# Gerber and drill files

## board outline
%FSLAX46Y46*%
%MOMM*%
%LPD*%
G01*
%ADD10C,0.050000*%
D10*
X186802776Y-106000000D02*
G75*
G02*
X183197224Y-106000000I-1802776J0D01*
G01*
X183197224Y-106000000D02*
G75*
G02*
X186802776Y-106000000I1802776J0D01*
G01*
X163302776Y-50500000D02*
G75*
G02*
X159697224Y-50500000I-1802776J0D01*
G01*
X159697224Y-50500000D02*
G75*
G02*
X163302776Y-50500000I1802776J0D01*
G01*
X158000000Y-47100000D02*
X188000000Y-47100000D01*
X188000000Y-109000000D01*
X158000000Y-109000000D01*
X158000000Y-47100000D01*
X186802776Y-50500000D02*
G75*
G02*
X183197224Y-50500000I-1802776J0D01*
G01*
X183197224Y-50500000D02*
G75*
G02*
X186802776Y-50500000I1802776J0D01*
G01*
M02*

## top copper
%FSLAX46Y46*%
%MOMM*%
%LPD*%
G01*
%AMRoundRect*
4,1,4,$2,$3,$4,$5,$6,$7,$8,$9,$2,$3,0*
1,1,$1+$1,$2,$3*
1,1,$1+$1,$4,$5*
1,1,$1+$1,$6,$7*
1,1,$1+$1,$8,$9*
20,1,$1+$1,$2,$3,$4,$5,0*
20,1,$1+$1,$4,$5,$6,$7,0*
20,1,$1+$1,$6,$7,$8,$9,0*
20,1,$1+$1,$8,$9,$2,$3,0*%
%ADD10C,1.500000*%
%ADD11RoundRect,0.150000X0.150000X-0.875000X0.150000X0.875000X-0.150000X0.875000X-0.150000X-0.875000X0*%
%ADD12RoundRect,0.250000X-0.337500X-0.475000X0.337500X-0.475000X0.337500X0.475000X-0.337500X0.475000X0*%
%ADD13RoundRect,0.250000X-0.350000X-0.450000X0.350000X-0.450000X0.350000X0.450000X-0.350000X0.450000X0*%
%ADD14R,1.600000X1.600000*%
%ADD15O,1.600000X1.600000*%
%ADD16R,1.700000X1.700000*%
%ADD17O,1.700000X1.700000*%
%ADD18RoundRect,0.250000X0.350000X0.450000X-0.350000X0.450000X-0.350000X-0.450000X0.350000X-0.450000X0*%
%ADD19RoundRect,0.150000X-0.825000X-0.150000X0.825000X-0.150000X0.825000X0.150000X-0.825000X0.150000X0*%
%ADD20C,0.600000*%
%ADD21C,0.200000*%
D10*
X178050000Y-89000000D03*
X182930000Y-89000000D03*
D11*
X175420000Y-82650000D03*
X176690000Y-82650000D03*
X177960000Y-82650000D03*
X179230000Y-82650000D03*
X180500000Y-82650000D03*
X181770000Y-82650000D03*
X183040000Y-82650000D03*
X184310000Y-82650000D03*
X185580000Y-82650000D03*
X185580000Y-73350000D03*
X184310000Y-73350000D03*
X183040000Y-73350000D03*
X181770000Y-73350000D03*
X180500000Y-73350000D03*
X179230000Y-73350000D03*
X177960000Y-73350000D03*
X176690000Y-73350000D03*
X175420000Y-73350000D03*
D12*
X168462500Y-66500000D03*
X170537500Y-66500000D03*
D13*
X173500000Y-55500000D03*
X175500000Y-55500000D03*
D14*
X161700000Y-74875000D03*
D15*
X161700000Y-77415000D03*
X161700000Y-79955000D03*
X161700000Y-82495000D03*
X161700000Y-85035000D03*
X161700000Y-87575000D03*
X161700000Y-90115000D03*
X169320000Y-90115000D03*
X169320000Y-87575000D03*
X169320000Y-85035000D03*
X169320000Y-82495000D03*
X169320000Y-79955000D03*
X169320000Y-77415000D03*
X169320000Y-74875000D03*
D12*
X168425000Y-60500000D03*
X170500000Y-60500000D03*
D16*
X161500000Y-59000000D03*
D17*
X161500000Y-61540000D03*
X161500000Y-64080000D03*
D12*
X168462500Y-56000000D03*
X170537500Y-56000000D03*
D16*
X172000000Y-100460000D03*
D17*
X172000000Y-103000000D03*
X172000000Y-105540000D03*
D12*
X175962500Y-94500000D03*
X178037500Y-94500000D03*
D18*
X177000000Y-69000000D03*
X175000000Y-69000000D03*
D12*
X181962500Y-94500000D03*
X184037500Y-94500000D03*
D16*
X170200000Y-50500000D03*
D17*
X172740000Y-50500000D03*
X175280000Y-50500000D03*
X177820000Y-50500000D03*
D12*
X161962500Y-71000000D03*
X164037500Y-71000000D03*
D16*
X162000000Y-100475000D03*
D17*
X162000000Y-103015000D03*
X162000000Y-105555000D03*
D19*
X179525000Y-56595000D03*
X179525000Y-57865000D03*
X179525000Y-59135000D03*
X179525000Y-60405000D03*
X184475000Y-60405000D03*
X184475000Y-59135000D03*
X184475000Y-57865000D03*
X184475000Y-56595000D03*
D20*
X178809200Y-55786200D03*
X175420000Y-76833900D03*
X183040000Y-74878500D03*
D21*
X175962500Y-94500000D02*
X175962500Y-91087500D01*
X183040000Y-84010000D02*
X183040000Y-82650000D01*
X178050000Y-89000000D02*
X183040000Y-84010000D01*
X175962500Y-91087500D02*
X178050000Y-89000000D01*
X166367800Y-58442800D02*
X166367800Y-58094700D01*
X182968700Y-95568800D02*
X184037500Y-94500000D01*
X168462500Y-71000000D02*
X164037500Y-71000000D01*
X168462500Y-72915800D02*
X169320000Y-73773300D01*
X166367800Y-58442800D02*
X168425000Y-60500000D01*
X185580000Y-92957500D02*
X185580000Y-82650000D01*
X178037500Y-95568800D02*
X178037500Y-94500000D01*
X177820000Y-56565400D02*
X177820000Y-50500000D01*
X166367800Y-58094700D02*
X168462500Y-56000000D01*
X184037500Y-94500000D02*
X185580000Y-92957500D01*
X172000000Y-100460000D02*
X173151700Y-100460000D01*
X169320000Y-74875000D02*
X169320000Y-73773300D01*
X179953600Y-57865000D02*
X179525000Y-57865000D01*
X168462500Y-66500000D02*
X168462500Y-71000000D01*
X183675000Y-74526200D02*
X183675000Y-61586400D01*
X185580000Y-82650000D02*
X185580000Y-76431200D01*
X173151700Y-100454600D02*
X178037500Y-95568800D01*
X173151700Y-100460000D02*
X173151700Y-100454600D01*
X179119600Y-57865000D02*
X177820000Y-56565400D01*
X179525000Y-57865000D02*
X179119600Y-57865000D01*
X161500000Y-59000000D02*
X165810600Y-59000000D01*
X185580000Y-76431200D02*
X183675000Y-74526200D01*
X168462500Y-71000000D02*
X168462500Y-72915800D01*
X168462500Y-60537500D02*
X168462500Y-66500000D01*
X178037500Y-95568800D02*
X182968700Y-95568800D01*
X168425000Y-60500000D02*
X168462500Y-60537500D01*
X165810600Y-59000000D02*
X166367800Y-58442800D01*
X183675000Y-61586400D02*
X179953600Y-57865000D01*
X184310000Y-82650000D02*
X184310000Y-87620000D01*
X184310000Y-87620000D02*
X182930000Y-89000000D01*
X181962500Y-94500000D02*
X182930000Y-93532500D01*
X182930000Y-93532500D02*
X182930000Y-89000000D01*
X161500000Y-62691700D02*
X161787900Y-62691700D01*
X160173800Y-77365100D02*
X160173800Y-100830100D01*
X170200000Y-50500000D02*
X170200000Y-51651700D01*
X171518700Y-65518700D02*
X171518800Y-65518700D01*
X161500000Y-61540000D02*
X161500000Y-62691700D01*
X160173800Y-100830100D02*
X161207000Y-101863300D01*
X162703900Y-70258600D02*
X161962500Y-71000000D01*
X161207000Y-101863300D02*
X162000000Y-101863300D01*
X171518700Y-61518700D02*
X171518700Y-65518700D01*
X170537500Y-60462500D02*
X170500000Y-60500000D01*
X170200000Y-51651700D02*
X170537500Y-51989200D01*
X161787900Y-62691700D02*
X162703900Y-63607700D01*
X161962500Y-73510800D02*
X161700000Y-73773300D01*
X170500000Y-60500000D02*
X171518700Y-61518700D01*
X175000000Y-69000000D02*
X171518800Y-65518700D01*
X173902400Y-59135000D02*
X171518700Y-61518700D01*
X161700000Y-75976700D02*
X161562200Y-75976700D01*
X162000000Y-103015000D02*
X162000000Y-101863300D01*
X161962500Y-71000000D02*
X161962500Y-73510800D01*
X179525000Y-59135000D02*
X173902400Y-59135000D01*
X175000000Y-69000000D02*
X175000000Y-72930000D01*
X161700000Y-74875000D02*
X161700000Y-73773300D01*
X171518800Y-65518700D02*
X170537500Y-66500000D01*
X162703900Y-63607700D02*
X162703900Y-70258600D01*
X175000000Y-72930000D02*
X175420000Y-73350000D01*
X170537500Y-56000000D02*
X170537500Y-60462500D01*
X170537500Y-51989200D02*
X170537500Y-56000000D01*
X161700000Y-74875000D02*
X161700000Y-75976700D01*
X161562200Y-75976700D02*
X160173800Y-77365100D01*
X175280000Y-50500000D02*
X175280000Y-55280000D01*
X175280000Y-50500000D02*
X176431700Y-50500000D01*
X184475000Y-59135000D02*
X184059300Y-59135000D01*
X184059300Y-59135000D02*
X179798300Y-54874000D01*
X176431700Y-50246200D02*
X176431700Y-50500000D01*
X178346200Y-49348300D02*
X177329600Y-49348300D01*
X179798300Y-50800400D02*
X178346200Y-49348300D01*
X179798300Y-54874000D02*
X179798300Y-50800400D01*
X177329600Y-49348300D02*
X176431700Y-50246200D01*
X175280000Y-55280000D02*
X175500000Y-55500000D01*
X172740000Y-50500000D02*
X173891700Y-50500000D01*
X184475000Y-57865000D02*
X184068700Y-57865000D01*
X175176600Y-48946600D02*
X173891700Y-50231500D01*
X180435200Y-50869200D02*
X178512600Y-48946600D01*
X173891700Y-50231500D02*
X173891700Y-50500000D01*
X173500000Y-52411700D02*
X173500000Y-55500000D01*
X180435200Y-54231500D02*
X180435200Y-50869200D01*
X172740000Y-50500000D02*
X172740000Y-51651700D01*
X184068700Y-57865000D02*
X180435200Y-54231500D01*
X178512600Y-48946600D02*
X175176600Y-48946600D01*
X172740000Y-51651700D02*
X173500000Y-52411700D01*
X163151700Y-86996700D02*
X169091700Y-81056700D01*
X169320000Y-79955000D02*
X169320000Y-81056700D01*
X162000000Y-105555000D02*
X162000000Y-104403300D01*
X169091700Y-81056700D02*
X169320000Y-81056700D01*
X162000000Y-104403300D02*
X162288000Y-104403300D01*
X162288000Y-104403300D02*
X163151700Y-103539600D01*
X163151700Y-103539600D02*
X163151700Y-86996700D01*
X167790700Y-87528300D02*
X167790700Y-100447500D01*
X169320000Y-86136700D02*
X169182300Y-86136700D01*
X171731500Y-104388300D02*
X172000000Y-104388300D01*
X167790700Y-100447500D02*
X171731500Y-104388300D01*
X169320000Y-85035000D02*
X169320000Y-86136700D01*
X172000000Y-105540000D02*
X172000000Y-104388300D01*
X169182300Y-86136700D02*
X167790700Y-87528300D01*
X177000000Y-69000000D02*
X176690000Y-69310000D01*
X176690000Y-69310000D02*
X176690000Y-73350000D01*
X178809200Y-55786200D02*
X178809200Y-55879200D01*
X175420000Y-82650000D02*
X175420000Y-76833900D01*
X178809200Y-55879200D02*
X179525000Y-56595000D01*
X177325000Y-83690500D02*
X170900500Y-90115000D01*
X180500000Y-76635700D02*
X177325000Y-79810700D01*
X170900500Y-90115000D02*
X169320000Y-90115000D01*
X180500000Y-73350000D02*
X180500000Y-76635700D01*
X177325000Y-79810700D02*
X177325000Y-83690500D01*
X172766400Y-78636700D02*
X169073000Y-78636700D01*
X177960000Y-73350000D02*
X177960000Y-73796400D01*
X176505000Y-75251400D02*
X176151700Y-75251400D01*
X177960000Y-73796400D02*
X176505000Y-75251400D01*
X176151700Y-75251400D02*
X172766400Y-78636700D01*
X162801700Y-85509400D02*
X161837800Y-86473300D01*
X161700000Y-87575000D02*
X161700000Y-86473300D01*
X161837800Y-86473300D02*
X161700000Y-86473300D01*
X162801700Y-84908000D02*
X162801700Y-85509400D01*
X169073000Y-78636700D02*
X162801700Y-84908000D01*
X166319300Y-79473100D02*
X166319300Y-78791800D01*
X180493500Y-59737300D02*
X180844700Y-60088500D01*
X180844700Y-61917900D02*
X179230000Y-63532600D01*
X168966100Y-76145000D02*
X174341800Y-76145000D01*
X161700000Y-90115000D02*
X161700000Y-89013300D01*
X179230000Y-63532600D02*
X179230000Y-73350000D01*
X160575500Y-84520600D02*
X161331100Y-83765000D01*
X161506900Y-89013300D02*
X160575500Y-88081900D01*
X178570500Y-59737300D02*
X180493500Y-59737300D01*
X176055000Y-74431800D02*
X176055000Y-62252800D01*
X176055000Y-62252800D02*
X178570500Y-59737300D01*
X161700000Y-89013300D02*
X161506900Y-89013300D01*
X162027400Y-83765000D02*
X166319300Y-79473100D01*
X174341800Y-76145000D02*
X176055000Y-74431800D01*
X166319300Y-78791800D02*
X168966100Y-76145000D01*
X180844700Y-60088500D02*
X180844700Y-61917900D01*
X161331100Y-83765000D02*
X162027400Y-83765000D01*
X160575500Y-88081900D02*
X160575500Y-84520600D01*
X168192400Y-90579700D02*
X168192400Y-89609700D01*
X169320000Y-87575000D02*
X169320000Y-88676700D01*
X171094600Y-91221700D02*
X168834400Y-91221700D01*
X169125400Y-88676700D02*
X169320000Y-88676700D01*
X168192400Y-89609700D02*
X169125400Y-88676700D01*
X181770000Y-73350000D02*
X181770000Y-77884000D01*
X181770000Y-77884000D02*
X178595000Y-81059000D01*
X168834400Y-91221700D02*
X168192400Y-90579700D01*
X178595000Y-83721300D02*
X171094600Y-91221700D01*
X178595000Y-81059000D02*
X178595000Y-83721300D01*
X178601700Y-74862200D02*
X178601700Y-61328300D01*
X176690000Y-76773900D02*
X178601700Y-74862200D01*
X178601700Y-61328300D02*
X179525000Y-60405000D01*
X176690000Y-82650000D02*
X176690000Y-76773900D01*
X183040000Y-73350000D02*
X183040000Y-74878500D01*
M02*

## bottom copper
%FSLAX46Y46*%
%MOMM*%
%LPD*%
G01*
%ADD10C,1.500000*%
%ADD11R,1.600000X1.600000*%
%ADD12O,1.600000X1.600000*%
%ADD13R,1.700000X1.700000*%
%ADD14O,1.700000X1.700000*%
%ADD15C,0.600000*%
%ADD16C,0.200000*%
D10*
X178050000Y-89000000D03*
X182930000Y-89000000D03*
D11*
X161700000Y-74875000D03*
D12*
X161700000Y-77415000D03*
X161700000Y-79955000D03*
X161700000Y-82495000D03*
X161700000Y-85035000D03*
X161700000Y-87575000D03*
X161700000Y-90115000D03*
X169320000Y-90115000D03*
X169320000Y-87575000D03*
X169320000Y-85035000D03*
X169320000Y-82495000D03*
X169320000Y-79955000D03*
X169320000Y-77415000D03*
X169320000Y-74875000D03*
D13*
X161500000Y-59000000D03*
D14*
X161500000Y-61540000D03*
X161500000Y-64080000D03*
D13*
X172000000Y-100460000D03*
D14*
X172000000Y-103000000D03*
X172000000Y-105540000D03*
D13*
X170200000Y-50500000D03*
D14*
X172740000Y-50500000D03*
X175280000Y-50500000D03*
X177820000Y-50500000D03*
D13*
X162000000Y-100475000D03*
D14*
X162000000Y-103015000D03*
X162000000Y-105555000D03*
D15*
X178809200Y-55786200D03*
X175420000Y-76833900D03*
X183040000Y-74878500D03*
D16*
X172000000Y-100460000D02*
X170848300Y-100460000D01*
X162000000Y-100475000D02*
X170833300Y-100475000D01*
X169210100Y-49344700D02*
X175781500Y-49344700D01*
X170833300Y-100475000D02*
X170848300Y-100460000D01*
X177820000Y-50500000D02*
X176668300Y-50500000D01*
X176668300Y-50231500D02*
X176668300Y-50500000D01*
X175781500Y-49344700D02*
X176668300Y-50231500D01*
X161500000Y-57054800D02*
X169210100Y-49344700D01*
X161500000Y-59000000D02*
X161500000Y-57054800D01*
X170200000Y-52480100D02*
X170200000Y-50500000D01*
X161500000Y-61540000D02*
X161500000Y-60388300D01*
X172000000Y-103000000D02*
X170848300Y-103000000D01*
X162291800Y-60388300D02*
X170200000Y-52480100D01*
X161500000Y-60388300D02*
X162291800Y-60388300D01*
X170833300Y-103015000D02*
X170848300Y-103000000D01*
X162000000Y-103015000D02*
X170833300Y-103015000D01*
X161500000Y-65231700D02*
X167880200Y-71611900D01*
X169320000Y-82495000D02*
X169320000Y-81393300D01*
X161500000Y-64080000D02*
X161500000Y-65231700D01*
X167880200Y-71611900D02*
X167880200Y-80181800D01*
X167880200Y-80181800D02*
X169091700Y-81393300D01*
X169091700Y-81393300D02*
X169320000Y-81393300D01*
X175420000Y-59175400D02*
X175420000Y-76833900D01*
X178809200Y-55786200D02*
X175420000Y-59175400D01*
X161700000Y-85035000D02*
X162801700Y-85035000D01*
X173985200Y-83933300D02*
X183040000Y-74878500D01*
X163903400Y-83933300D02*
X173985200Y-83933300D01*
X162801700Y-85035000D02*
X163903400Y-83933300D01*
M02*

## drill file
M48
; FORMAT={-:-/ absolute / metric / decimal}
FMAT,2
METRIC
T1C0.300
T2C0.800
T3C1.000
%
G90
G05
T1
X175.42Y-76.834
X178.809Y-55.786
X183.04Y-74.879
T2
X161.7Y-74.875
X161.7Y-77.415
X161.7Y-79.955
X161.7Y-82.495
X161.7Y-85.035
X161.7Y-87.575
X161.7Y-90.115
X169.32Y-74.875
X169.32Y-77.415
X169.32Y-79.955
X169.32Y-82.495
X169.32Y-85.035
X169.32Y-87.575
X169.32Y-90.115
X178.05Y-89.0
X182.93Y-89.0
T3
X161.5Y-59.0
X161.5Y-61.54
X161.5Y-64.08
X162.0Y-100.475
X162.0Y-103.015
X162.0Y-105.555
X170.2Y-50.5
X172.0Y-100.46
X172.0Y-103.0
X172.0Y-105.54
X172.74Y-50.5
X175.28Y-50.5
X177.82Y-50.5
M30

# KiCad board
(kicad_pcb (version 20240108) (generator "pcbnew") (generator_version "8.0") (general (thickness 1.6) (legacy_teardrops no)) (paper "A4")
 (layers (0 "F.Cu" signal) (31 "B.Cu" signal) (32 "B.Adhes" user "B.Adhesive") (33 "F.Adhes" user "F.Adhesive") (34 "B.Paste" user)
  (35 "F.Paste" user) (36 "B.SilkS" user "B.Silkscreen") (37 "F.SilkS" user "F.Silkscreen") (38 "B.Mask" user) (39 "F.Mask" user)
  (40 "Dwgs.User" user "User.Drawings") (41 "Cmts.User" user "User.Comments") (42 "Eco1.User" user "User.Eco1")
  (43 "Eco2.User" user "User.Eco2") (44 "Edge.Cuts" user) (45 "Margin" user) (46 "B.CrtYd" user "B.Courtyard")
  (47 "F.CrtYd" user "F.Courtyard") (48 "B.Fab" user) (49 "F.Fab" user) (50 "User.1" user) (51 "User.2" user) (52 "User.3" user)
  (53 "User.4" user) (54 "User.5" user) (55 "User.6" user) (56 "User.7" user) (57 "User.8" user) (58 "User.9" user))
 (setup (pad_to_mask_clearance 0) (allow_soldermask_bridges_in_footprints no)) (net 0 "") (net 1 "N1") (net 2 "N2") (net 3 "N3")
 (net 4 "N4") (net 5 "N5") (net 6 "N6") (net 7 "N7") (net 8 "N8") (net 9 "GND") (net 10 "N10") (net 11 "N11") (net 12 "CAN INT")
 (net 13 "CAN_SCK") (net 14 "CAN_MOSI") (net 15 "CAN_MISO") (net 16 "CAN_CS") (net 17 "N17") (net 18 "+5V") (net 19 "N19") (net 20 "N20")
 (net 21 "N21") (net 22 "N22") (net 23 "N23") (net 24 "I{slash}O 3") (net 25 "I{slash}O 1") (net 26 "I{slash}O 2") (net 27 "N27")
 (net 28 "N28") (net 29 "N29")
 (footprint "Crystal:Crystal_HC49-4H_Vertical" (layer "F.Cu") (at 178.05 89)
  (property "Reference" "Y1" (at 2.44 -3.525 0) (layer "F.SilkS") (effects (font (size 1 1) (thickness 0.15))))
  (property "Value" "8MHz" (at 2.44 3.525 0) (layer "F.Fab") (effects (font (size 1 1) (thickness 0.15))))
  (pad "1" thru_hole circle (at 0 0) (size 1.5 1.5) (drill 0.8) (layers "*.Cu" "*.Mask") (remove_unused_layers no) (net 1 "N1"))
  (pad "2" thru_hole circle (at 4.88 0) (size 1.5 1.5) (drill 0.8) (layers "*.Cu" "*.Mask") (remove_unused_layers no) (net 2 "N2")))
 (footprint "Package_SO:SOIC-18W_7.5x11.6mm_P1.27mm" (layer "F.Cu") (at 180.5 78 90)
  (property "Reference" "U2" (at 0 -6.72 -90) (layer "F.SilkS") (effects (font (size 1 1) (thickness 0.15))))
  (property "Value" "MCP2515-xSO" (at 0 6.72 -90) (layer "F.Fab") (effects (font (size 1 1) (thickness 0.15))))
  (pad "1" smd roundrect (at -4.65 -5.08 90) (size 2.05 0.6) (layers "F.Cu" "F.Paste" "F.Mask") (roundrect_rratio 0.25) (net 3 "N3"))
  (pad "2" smd roundrect (at -4.65 -3.81 90) (size 2.05 0.6) (layers "F.Cu" "F.Paste" "F.Mask") (roundrect_rratio 0.25) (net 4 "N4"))
  (pad "3" smd roundrect (at -4.65 -2.54 90) (size 2.05 0.6) (layers "F.Cu" "F.Paste" "F.Mask") (roundrect_rratio 0.25) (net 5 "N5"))
  (pad "4" smd roundrect (at -4.65 -1.27 90) (size 2.05 0.6) (layers "F.Cu" "F.Paste" "F.Mask") (roundrect_rratio 0.25) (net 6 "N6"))
  (pad "5" smd roundrect (at -4.65 0 90) (size 2.05 0.6) (layers "F.Cu" "F.Paste" "F.Mask") (roundrect_rratio 0.25) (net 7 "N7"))
  (pad "6" smd roundrect (at -4.65 1.27 90) (size 2.05 0.6) (layers "F.Cu" "F.Paste" "F.Mask") (roundrect_rratio 0.25) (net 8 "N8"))
  (pad "7" smd roundrect (at -4.65 2.54 90) (size 2.05 0.6) (layers "F.Cu" "F.Paste" "F.Mask") (roundrect_rratio 0.25) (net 1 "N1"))
  (pad "8" smd roundrect (at -4.65 3.81 90) (size 2.05 0.6) (layers "F.Cu" "F.Paste" "F.Mask") (roundrect_rratio 0.25) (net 2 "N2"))
  (pad "9" smd roundrect (at -4.65 5.08 90) (size 2.05 0.6) (layers "F.Cu" "F.Paste" "F.Mask") (roundrect_rratio 0.25) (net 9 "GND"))
  (pad "10" smd roundrect (at 4.65 5.08 90) (size 2.05 0.6) (layers "F.Cu" "F.Paste" "F.Mask") (roundrect_rratio 0.25) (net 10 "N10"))
  (pad "11" smd roundrect (at 4.65 3.81 90) (size 2.05 0.6) (layers "F.Cu" "F.Paste" "F.Mask") (roundrect_rratio 0.25) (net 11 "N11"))
  (pad "12" smd roundrect (at 4.65 2.54 90) (size 2.05 0.6) (layers "F.Cu" "F.Paste" "F.Mask") (roundrect_rratio 0.25) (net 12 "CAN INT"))
  (pad "13" smd roundrect (at 4.65 1.27 90) (size 2.05 0.6) (layers "F.Cu" "F.Paste" "F.Mask") (roundrect_rratio 0.25) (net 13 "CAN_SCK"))
  (pad "14" smd roundrect (at 4.65 0 90) (size 2.05 0.6) (layers "F.Cu" "F.Paste" "F.Mask") (roundrect_rratio 0.25) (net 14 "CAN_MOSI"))
  (pad "15" smd roundrect (at 4.65 -1.27 90) (size 2.05 0.6) (layers "F.Cu" "F.Paste" "F.Mask") (roundrect_rratio 0.25) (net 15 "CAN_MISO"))
  (pad "16" smd roundrect (at 4.65 -2.54 90) (size 2.05 0.6) (layers "F.Cu" "F.Paste" "F.Mask") (roundrect_rratio 0.25) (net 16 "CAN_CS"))
  (pad "17" smd roundrect (at 4.65 -3.81 90) (size 2.05 0.6) (layers "F.Cu" "F.Paste" "F.Mask") (roundrect_rratio 0.25) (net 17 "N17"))
  (pad "18" smd roundrect (at 4.65 -5.08 90) (size 2.05 0.6) (layers "F.Cu" "F.Paste" "F.Mask") (roundrect_rratio 0.25) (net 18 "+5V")))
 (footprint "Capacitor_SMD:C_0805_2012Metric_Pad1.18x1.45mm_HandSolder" (layer "F.Cu") (at 169.5 66.5)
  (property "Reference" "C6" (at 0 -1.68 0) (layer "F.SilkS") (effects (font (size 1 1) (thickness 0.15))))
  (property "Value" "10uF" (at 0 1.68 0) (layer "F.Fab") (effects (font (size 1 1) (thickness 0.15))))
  (pad "1" smd roundrect (at -1.0375 0) (size 1.175 1.45) (layers "F.Cu" "F.Paste" "F.Mask") (roundrect_rratio 0.212766) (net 9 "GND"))
  (pad "2" smd roundrect (at 1.0375 0) (size 1.175 1.45) (layers "F.Cu" "F.Paste" "F.Mask") (roundrect_rratio 0.212766) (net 18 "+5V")))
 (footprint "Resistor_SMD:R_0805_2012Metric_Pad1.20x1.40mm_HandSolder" (layer "F.Cu") (at 174.5 55.5)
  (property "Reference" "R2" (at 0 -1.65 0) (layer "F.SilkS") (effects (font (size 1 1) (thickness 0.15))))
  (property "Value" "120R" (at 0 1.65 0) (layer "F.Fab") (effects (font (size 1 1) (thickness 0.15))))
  (pad "1" smd roundrect (at -1 0) (size 1.2 1.4) (layers "F.Cu" "F.Paste" "F.Mask") (roundrect_rratio 0.208333) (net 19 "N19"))
  (pad "2" smd roundrect (at 1 0) (size 1.2 1.4) (layers "F.Cu" "F.Paste" "F.Mask") (roundrect_rratio 0.208333) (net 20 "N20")))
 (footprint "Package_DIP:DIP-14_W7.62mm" (layer "F.Cu") (at 161.7 74.875)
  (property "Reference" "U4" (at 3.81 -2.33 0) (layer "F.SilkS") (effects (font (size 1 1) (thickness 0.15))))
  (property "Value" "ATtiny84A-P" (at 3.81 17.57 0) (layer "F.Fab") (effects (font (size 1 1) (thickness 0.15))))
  (pad "1" thru_hole rect (at 0 0) (size 1.6 1.6) (drill 0.8) (layers "*.Cu" "*.Mask") (remove_unused_layers no) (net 18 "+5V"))
  (pad "2" thru_hole oval (at 0 2.54) (size 1.6 1.6) (drill 0.8) (layers "*.Cu" "*.Mask") (remove_unused_layers no) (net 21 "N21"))
  (pad "3" thru_hole oval (at 0 5.08) (size 1.6 1.6) (drill 0.8) (layers "*.Cu" "*.Mask") (remove_unused_layers no) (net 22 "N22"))
  (pad "4" thru_hole oval (at 0 7.62) (size 1.6 1.6) (drill 0.8) (layers "*.Cu" "*.Mask") (remove_unused_layers no) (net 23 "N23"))
  (pad "5" thru_hole oval (at 0 10.16) (size 1.6 1.6) (drill 0.8) (layers "*.Cu" "*.Mask") (remove_unused_layers no) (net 12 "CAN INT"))
  (pad "6" thru_hole oval (at 0 12.7) (size 1.6 1.6) (drill 0.8) (layers "*.Cu" "*.Mask") (remove_unused_layers no) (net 16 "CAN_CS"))
  (pad "7" thru_hole oval (at 0 15.24) (size 1.6 1.6) (drill 0.8) (layers "*.Cu" "*.Mask") (remove_unused_layers no) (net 15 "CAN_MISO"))
  (pad "8" thru_hole oval (at 7.62 15.24) (size 1.6 1.6) (drill 0.8) (layers "*.Cu" "*.Mask") (remove_unused_layers no) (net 14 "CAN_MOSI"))
  (pad "9" thru_hole oval (at 7.62 12.7) (size 1.6 1.6) (drill 0.8) (layers "*.Cu" "*.Mask") (remove_unused_layers no) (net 13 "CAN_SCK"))
  (pad "10" thru_hole oval (at 7.62 10.16) (size 1.6 1.6) (drill 0.8) (layers "*.Cu" "*.Mask") (remove_unused_layers no)
   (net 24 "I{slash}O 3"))
  (pad "11" thru_hole oval (at 7.62 7.62) (size 1.6 1.6) (drill 0.8) (layers "*.Cu" "*.Mask") (remove_unused_layers no)
   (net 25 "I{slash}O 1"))
  (pad "12" thru_hole oval (at 7.62 5.08) (size 1.6 1.6) (drill 0.8) (layers "*.Cu" "*.Mask") (remove_unused_layers no)
   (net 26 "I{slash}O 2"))
  (pad "13" thru_hole oval (at 7.62 2.54) (size 1.6 1.6) (drill 0.8) (layers "*.Cu" "*.Mask") (remove_unused_layers no) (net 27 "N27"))
  (pad "14" thru_hole oval (at 7.62 0) (size 1.6 1.6) (drill 0.8) (layers "*.Cu" "*.Mask") (remove_unused_layers no) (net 9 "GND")))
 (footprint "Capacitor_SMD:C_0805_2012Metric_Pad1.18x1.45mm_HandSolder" (layer "F.Cu") (at 169.4625 60.5)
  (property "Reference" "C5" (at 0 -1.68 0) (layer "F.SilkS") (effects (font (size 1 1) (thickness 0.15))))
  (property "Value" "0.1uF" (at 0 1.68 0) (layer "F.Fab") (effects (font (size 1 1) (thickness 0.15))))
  (pad "1" smd roundrect (at -1.0375 0) (size 1.175 1.45) (layers "F.Cu" "F.Paste" "F.Mask") (roundrect_rratio 0.212766) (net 9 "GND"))
  (pad "2" smd roundrect (at 1.0375 0) (size 1.175 1.45) (layers "F.Cu" "F.Paste" "F.Mask") (roundrect_rratio 0.212766) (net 18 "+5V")))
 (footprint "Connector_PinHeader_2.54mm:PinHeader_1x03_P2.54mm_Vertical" (layer "F.Cu") (at 161.5 59)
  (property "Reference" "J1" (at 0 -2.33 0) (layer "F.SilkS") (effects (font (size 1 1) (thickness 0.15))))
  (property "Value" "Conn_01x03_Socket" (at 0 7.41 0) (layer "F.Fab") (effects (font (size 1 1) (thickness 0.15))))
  (pad "1" thru_hole rect (at 0 0) (size 1.7 1.7) (drill 1) (layers "*.Cu" "*.Mask") (remove_unused_layers no) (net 9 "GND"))
  (pad "2" thru_hole oval (at 0 2.54) (size 1.7 1.7) (drill 1) (layers "*.Cu" "*.Mask") (remove_unused_layers no) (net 18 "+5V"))
  (pad "3" thru_hole oval (at 0 5.08) (size 1.7 1.7) (drill 1) (layers "*.Cu" "*.Mask") (remove_unused_layers no) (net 25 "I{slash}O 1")))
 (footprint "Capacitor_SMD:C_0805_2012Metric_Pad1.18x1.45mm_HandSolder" (layer "F.Cu") (at 169.5 56)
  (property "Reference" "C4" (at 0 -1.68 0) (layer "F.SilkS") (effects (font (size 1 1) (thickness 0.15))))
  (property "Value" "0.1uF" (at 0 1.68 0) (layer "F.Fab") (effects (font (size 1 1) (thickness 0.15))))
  (pad "1" smd roundrect (at -1.0375 0) (size 1.175 1.45) (layers "F.Cu" "F.Paste" "F.Mask") (roundrect_rratio 0.212766) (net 9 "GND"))
  (pad "2" smd roundrect (at 1.0375 0) (size 1.175 1.45) (layers "F.Cu" "F.Paste" "F.Mask") (roundrect_rratio 0.212766) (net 18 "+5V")))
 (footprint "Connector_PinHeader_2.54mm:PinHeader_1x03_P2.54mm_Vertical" (layer "F.Cu") (at 172 100.46)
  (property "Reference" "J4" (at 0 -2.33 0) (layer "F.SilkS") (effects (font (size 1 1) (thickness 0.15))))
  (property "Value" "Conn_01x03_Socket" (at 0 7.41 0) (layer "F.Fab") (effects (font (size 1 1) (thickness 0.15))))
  (pad "1" thru_hole rect (at 0 0) (size 1.7 1.7) (drill 1) (layers "*.Cu" "*.Mask") (remove_unused_layers no) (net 9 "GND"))
  (pad "2" thru_hole oval (at 0 2.54) (size 1.7 1.7) (drill 1) (layers "*.Cu" "*.Mask") (remove_unused_layers no) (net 18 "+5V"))
  (pad "3" thru_hole oval (at 0 5.08) (size 1.7 1.7) (drill 1) (layers "*.Cu" "*.Mask") (remove_unused_layers no) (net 24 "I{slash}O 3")))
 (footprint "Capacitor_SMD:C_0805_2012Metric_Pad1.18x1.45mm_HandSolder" (layer "F.Cu") (at 177 94.5)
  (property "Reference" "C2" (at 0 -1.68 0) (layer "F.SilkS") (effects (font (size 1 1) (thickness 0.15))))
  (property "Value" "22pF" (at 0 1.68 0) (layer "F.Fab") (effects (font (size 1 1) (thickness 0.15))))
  (pad "1" smd roundrect (at -1.0375 0) (size 1.175 1.45) (layers "F.Cu" "F.Paste" "F.Mask") (roundrect_rratio 0.212766) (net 1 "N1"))
  (pad "2" smd roundrect (at 1.0375 0) (size 1.175 1.45) (layers "F.Cu" "F.Paste" "F.Mask") (roundrect_rratio 0.212766) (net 9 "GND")))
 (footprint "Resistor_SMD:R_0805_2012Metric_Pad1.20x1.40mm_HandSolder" (layer "F.Cu") (at 176 69 180)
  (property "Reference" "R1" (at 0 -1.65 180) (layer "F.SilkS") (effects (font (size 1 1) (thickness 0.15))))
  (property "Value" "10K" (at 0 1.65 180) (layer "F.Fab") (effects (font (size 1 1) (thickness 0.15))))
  (pad "1" smd roundrect (at -1 0 180) (size 1.2 1.4) (layers "F.Cu" "F.Paste" "F.Mask") (roundrect_rratio 0.208333) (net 17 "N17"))
  (pad "2" smd roundrect (at 1 0 180) (size 1.2 1.4) (layers "F.Cu" "F.Paste" "F.Mask") (roundrect_rratio 0.208333) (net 18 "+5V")))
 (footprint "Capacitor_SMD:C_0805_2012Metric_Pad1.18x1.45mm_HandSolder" (layer "F.Cu") (at 183 94.5)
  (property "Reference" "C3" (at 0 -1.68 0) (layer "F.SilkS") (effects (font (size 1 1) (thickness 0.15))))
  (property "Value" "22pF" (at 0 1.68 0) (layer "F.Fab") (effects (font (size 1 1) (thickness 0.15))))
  (pad "1" smd roundrect (at -1.0375 0) (size 1.175 1.45) (layers "F.Cu" "F.Paste" "F.Mask") (roundrect_rratio 0.212766) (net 2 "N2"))
  (pad "2" smd roundrect (at 1.0375 0) (size 1.175 1.45) (layers "F.Cu" "F.Paste" "F.Mask") (roundrect_rratio 0.212766) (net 9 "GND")))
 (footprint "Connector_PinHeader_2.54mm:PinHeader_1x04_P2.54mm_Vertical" (layer "F.Cu") (at 170.2 50.5 90)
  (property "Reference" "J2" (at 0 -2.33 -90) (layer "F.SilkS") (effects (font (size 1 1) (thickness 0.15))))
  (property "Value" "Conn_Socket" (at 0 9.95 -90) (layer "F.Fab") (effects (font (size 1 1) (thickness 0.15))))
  (pad "1" thru_hole rect (at 0 0 90) (size 1.7 1.7) (drill 1) (layers "*.Cu" "*.Mask") (remove_unused_layers no) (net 18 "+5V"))
  (pad "2" thru_hole oval (at 0 2.54 90) (size 1.7 1.7) (drill 1) (layers "*.Cu" "*.Mask") (remove_unused_layers no) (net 19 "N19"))
  (pad "3" thru_hole oval (at 0 5.08 90) (size 1.7 1.7) (drill 1) (layers "*.Cu" "*.Mask") (remove_unused_layers no) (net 20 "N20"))
  (pad "4" thru_hole oval (at 0 7.62 90) (size 1.7 1.7) (drill 1) (layers "*.Cu" "*.Mask") (remove_unused_layers no) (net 9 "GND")))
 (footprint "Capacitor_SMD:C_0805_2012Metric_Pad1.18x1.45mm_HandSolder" (layer "F.Cu") (at 163 71)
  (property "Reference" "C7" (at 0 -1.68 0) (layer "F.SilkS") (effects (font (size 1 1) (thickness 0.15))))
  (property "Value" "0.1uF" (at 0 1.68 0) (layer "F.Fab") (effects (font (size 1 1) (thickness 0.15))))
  (pad "1" smd roundrect (at -1.0375 0) (size 1.175 1.45) (layers "F.Cu" "F.Paste" "F.Mask") (roundrect_rratio 0.212766) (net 18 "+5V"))
  (pad "2" smd roundrect (at 1.0375 0) (size 1.175 1.45) (layers "F.Cu" "F.Paste" "F.Mask") (roundrect_rratio 0.212766) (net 9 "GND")))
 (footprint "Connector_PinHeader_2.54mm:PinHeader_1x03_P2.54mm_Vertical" (layer "F.Cu") (at 162 100.475)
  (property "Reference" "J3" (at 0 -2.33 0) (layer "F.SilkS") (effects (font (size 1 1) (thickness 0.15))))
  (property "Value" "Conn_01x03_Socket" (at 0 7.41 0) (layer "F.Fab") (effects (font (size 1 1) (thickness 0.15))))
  (pad "1" thru_hole rect (at 0 0) (size 1.7 1.7) (drill 1) (layers "*.Cu" "*.Mask") (remove_unused_layers no) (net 9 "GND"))
  (pad "2" thru_hole oval (at 0 2.54) (size 1.7 1.7) (drill 1) (layers "*.Cu" "*.Mask") (remove_unused_layers no) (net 18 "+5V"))
  (pad "3" thru_hole oval (at 0 5.08) (size 1.7 1.7) (drill 1) (layers "*.Cu" "*.Mask") (remove_unused_layers no) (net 26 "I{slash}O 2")))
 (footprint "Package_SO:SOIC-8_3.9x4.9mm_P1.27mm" (layer "F.Cu") (at 182 58.5)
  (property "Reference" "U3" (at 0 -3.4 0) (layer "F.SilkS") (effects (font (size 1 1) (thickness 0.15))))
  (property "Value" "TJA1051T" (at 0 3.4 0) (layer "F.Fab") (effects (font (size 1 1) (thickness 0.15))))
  (pad "1" smd roundrect (at -2.475 -1.905) (size 1.95 0.6) (layers "F.Cu" "F.Paste" "F.Mask") (roundrect_rratio 0.25) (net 3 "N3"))
  (pad "2" smd roundrect (at -2.475 -0.635) (size 1.95 0.6) (layers "F.Cu" "F.Paste" "F.Mask") (roundrect_rratio 0.25) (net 9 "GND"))
  (pad "3" smd roundrect (at -2.475 0.635) (size 1.95 0.6) (layers "F.Cu" "F.Paste" "F.Mask") (roundrect_rratio 0.25) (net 18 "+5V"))
  (pad "4" smd roundrect (at -2.475 1.905) (size 1.95 0.6) (layers "F.Cu" "F.Paste" "F.Mask") (roundrect_rratio 0.25) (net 4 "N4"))
  (pad "5" smd roundrect (at 2.475 1.905) (size 1.95 0.6) (layers "F.Cu" "F.Paste" "F.Mask") (roundrect_rratio 0.25) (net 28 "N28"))
  (pad "6" smd roundrect (at 2.475 0.635) (size 1.95 0.6) (layers "F.Cu" "F.Paste" "F.Mask") (roundrect_rratio 0.25) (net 20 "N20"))
  (pad "7" smd roundrect (at 2.475 -0.635) (size 1.95 0.6) (layers "F.Cu" "F.Paste" "F.Mask") (roundrect_rratio 0.25) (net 19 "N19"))
  (pad "8" smd roundrect (at 2.475 -1.905) (size 1.95 0.6) (layers "F.Cu" "F.Paste" "F.Mask") (roundrect_rratio 0.25) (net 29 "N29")))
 (gr_circle (center 185 106) (end 186 107.5) (stroke (width 0.05) (type default)) (fill none) (layer "Edge.Cuts"))
 (gr_circle (center 161.5 50.5) (end 162.5 52) (stroke (width 0.05) (type default)) (fill none) (layer "Edge.Cuts"))
 (gr_rect (start 158 47.1) (end 188 109) (stroke (width 0.05) (type default)) (fill none) (layer "Edge.Cuts"))
 (gr_circle (center 185 50.5) (end 186 52) (stroke (width 0.05) (type default)) (fill none) (layer "Edge.Cuts"))
 (segment (start 175.9625 94.5) (end 175.9625 91.0875) (width 0.2) (layer "F.Cu") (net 1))
 (segment (start 183.04 84.01) (end 183.04 82.65) (width 0.2) (layer "F.Cu") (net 1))
 (segment (start 178.05 89) (end 183.04 84.01) (width 0.2) (layer "F.Cu") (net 1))
 (segment (start 175.9625 91.0875) (end 178.05 89) (width 0.2) (layer "F.Cu") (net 1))
 (segment (start 166.3678 58.4428) (end 166.3678 58.0947) (width 0.2) (layer "F.Cu") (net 9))
 (segment (start 182.9687 95.5688) (end 184.0375 94.5) (width 0.2) (layer "F.Cu") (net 9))
 (segment (start 168.4625 71) (end 164.0375 71) (width 0.2) (layer "F.Cu") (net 9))
 (segment (start 168.4625 72.9158) (end 169.32 73.7733) (width 0.2) (layer "F.Cu") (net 9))
 (segment (start 166.3678 58.4428) (end 168.425 60.5) (width 0.2) (layer "F.Cu") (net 9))
 (segment (start 185.58 92.9575) (end 185.58 82.65) (width 0.2) (layer "F.Cu") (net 9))
 (segment (start 178.0375 95.5688) (end 178.0375 94.5) (width 0.2) (layer "F.Cu") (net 9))
 (segment (start 177.82 56.5654) (end 177.82 50.5) (width 0.2) (layer "F.Cu") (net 9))
 (segment (start 166.3678 58.0947) (end 168.4625 56) (width 0.2) (layer "F.Cu") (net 9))
 (segment (start 184.0375 94.5) (end 185.58 92.9575) (width 0.2) (layer "F.Cu") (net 9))
 (segment (start 172 100.46) (end 173.1517 100.46) (width 0.2) (layer "F.Cu") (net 9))
 (segment (start 169.32 74.875) (end 169.32 73.7733) (width 0.2) (layer "F.Cu") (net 9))
 (segment (start 179.9536 57.865) (end 179.525 57.865) (width 0.2) (layer "F.Cu") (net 9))
 (segment (start 168.4625 66.5) (end 168.4625 71) (width 0.2) (layer "F.Cu") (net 9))
 (segment (start 183.675 74.5262) (end 183.675 61.5864) (width 0.2) (layer "F.Cu") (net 9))
 (segment (start 185.58 82.65) (end 185.58 76.4312) (width 0.2) (layer "F.Cu") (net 9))
 (segment (start 173.1517 100.4546) (end 178.0375 95.5688) (width 0.2) (layer "F.Cu") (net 9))
 (segment (start 173.1517 100.46) (end 173.1517 100.4546) (width 0.2) (layer "F.Cu") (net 9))
 (segment (start 179.1196 57.865) (end 177.82 56.5654) (width 0.2) (layer "F.Cu") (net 9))
 (segment (start 179.525 57.865) (end 179.1196 57.865) (width 0.2) (layer "F.Cu") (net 9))
 (segment (start 161.5 59) (end 165.8106 59) (width 0.2) (layer "F.Cu") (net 9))
 (segment (start 185.58 76.4312) (end 183.675 74.5262) (width 0.2) (layer "F.Cu") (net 9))
 (segment (start 168.4625 71) (end 168.4625 72.9158) (width 0.2) (layer "F.Cu") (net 9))
 (segment (start 168.4625 60.5375) (end 168.4625 66.5) (width 0.2) (layer "F.Cu") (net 9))
 (segment (start 178.0375 95.5688) (end 182.9687 95.5688) (width 0.2) (layer "F.Cu") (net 9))
 (segment (start 168.425 60.5) (end 168.4625 60.5375) (width 0.2) (layer "F.Cu") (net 9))
 (segment (start 165.8106 59) (end 166.3678 58.4428) (width 0.2) (layer "F.Cu") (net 9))
 (segment (start 183.675 61.5864) (end 179.9536 57.865) (width 0.2) (layer "F.Cu") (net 9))
 (segment (start 172 100.46) (end 170.8483 100.46) (width 0.2) (layer "B.Cu") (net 9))
 (segment (start 162 100.475) (end 170.8333 100.475) (width 0.2) (layer "B.Cu") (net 9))
 (segment (start 169.2101 49.3447) (end 175.7815 49.3447) (width 0.2) (layer "B.Cu") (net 9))
 (segment (start 170.8333 100.475) (end 170.8483 100.46) (width 0.2) (layer "B.Cu") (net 9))
 (segment (start 177.82 50.5) (end 176.6683 50.5) (width 0.2) (layer "B.Cu") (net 9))
 (segment (start 176.6683 50.2315) (end 176.6683 50.5) (width 0.2) (layer "B.Cu") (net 9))
 (segment (start 175.7815 49.3447) (end 176.6683 50.2315) (width 0.2) (layer "B.Cu") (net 9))
 (segment (start 161.5 57.0548) (end 169.2101 49.3447) (width 0.2) (layer "B.Cu") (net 9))
 (segment (start 161.5 59) (end 161.5 57.0548) (width 0.2) (layer "B.Cu") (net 9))
 (segment (start 184.31 82.65) (end 184.31 87.62) (width 0.2) (layer "F.Cu") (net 2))
 (segment (start 184.31 87.62) (end 182.93 89) (width 0.2) (layer "F.Cu") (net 2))
 (segment (start 181.9625 94.5) (end 182.93 93.5325) (width 0.2) (layer "F.Cu") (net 2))
 (segment (start 182.93 93.5325) (end 182.93 89) (width 0.2) (layer "F.Cu") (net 2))
 (segment (start 161.5 62.6917) (end 161.7879 62.6917) (width 0.2) (layer "F.Cu") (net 18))
 (segment (start 160.1738 77.3651) (end 160.1738 100.8301) (width 0.2) (layer "F.Cu") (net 18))
 (segment (start 170.2 50.5) (end 170.2 51.6517) (width 0.2) (layer "F.Cu") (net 18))
 (segment (start 171.5187 65.5187) (end 171.5188 65.5187) (width 0.2) (layer "F.Cu") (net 18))
 (segment (start 161.5 61.54) (end 161.5 62.6917) (width 0.2) (layer "F.Cu") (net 18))
 (segment (start 160.1738 100.8301) (end 161.207 101.8633) (width 0.2) (layer "F.Cu") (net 18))
 (segment (start 162.7039 70.2586) (end 161.9625 71) (width 0.2) (layer "F.Cu") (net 18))
 (segment (start 161.207 101.8633) (end 162 101.8633) (width 0.2) (layer "F.Cu") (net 18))
 (segment (start 171.5187 61.5187) (end 171.5187 65.5187) (width 0.2) (layer "F.Cu") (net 18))
 (segment (start 170.5375 60.4625) (end 170.5 60.5) (width 0.2) (layer "F.Cu") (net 18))
 (segment (start 170.2 51.6517) (end 170.5375 51.9892) (width 0.2) (layer "F.Cu") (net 18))
 (segment (start 161.7879 62.6917) (end 162.7039 63.6077) (width 0.2) (layer "F.Cu") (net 18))
 (segment (start 161.9625 73.5108) (end 161.7 73.7733) (width 0.2) (layer "F.Cu") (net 18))
 (segment (start 170.5 60.5) (end 171.5187 61.5187) (width 0.2) (layer "F.Cu") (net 18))
 (segment (start 175 69) (end 171.5188 65.5187) (width 0.2) (layer "F.Cu") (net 18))
 (segment (start 173.9024 59.135) (end 171.5187 61.5187) (width 0.2) (layer "F.Cu") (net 18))
 (segment (start 161.7 75.9767) (end 161.5622 75.9767) (width 0.2) (layer "F.Cu") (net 18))
 (segment (start 162 103.015) (end 162 101.8633) (width 0.2) (layer "F.Cu") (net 18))
 (segment (start 161.9625 71) (end 161.9625 73.5108) (width 0.2) (layer "F.Cu") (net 18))
 (segment (start 179.525 59.135) (end 173.9024 59.135) (width 0.2) (layer "F.Cu") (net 18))
 (segment (start 175 69) (end 175 72.93) (width 0.2) (layer "F.Cu") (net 18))
 (segment (start 161.7 74.875) (end 161.7 73.7733) (width 0.2) (layer "F.Cu") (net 18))
 (segment (start 171.5188 65.5187) (end 170.5375 66.5) (width 0.2) (layer "F.Cu") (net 18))
 (segment (start 162.7039 63.6077) (end 162.7039 70.2586) (width 0.2) (layer "F.Cu") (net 18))
 (segment (start 175 72.93) (end 175.42 73.35) (width 0.2) (layer "F.Cu") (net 18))
 (segment (start 170.5375 56) (end 170.5375 60.4625) (width 0.2) (layer "F.Cu") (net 18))
 (segment (start 170.5375 51.9892) (end 170.5375 56) (width 0.2) (layer "F.Cu") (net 18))
 (segment (start 161.7 74.875) (end 161.7 75.9767) (width 0.2) (layer "F.Cu") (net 18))
 (segment (start 161.5622 75.9767) (end 160.1738 77.3651) (width 0.2) (layer "F.Cu") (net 18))
 (segment (start 170.2 52.4801) (end 170.2 50.5) (width 0.2) (layer "B.Cu") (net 18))
 (segment (start 161.5 61.54) (end 161.5 60.3883) (width 0.2) (layer "B.Cu") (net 18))
 (segment (start 172 103) (end 170.8483 103) (width 0.2) (layer "B.Cu") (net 18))
 (segment (start 162.2918 60.3883) (end 170.2 52.4801) (width 0.2) (layer "B.Cu") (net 18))
 (segment (start 161.5 60.3883) (end 162.2918 60.3883) (width 0.2) (layer "B.Cu") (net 18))
 (segment (start 170.8333 103.015) (end 170.8483 103) (width 0.2) (layer "B.Cu") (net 18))
 (segment (start 162 103.015) (end 170.8333 103.015) (width 0.2) (layer "B.Cu") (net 18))
 (segment (start 161.5 65.2317) (end 167.8802 71.6119) (width 0.2) (layer "B.Cu") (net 25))
 (segment (start 169.32 82.495) (end 169.32 81.3933) (width 0.2) (layer "B.Cu") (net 25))
 (segment (start 161.5 64.08) (end 161.5 65.2317) (width 0.2) (layer "B.Cu") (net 25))
 (segment (start 167.8802 71.6119) (end 167.8802 80.1818) (width 0.2) (layer "B.Cu") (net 25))
 (segment (start 167.8802 80.1818) (end 169.0917 81.3933) (width 0.2) (layer "B.Cu") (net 25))
 (segment (start 169.0917 81.3933) (end 169.32 81.3933) (width 0.2) (layer "B.Cu") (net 25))
 (segment (start 175.28 50.5) (end 175.28 55.28) (width 0.2) (layer "F.Cu") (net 20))
 (segment (start 175.28 50.5) (end 176.4317 50.5) (width 0.2) (layer "F.Cu") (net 20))
 (segment (start 184.475 59.135) (end 184.0593 59.135) (width 0.2) (layer "F.Cu") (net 20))
 (segment (start 184.0593 59.135) (end 179.7983 54.874) (width 0.2) (layer "F.Cu") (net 20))
 (segment (start 176.4317 50.2462) (end 176.4317 50.5) (width 0.2) (layer "F.Cu") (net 20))
 (segment (start 178.3462 49.3483) (end 177.3296 49.3483) (width 0.2) (layer "F.Cu") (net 20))
 (segment (start 179.7983 50.8004) (end 178.3462 49.3483) (width 0.2) (layer "F.Cu") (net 20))
 (segment (start 179.7983 54.874) (end 179.7983 50.8004) (width 0.2) (layer "F.Cu") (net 20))
 (segment (start 177.3296 49.3483) (end 176.4317 50.2462) (width 0.2) (layer "F.Cu") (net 20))
 (segment (start 175.28 55.28) (end 175.5 55.5) (width 0.2) (layer "F.Cu") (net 20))
 (segment (start 172.74 50.5) (end 173.8917 50.5) (width 0.2) (layer "F.Cu") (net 19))
 (segment (start 184.475 57.865) (end 184.0687 57.865) (width 0.2) (layer "F.Cu") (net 19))
 (segment (start 175.1766 48.9466) (end 173.8917 50.2315) (width 0.2) (layer "F.Cu") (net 19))
 (segment (start 180.4352 50.8692) (end 178.5126 48.9466) (width 0.2) (layer "F.Cu") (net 19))
 (segment (start 173.8917 50.2315) (end 173.8917 50.5) (width 0.2) (layer "F.Cu") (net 19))
 (segment (start 173.5 52.4117) (end 173.5 55.5) (width 0.2) (layer "F.Cu") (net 19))
 (segment (start 180.4352 54.2315) (end 180.4352 50.8692) (width 0.2) (layer "F.Cu") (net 19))
 (segment (start 172.74 50.5) (end 172.74 51.6517) (width 0.2) (layer "F.Cu") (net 19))
 (segment (start 184.0687 57.865) (end 180.4352 54.2315) (width 0.2) (layer "F.Cu") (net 19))
 (segment (start 178.5126 48.9466) (end 175.1766 48.9466) (width 0.2) (layer "F.Cu") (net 19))
 (segment (start 172.74 51.6517) (end 173.5 52.4117) (width 0.2) (layer "F.Cu") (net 19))
 (segment (start 163.1517 86.9967) (end 169.0917 81.0567) (width 0.2) (layer "F.Cu") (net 26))
 (segment (start 169.32 79.955) (end 169.32 81.0567) (width 0.2) (layer "F.Cu") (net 26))
 (segment (start 162 105.555) (end 162 104.4033) (width 0.2) (layer "F.Cu") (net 26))
 (segment (start 169.0917 81.0567) (end 169.32 81.0567) (width 0.2) (layer "F.Cu") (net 26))
 (segment (start 162 104.4033) (end 162.288 104.4033) (width 0.2) (layer "F.Cu") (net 26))
 (segment (start 162.288 104.4033) (end 163.1517 103.5396) (width 0.2) (layer "F.Cu") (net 26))
 (segment (start 163.1517 103.5396) (end 163.1517 86.9967) (width 0.2) (layer "F.Cu") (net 26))
 (segment (start 167.7907 87.5283) (end 167.7907 100.4475) (width 0.2) (layer "F.Cu") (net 24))
 (segment (start 169.32 86.1367) (end 169.1823 86.1367) (width 0.2) (layer "F.Cu") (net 24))
 (segment (start 171.7315 104.3883) (end 172 104.3883) (width 0.2) (layer "F.Cu") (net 24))
 (segment (start 167.7907 100.4475) (end 171.7315 104.3883) (width 0.2) (layer "F.Cu") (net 24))
 (segment (start 169.32 85.035) (end 169.32 86.1367) (width 0.2) (layer "F.Cu") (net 24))
 (segment (start 172 105.54) (end 172 104.3883) (width 0.2) (layer "F.Cu") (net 24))
 (segment (start 169.1823 86.1367) (end 167.7907 87.5283) (width 0.2) (layer "F.Cu") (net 24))
 (segment (start 177 69) (end 176.69 69.31) (width 0.2) (layer "F.Cu") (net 17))
 (segment (start 176.69 69.31) (end 176.69 73.35) (width 0.2) (layer "F.Cu") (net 17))
 (segment (start 178.8092 55.7862) (end 178.8092 55.8792) (width 0.2) (layer "F.Cu") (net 3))
 (segment (start 175.42 82.65) (end 175.42 76.8339) (width 0.2) (layer "F.Cu") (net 3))
 (segment (start 178.8092 55.8792) (end 179.525 56.595) (width 0.2) (layer "F.Cu") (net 3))
 (via (at 178.8092 55.7862) (size 0.6) (drill 0.3) (layers "F.Cu" "B.Cu") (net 3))
 (via (at 175.42 76.8339) (size 0.6) (drill 0.3) (layers "F.Cu" "B.Cu") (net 3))
 (segment (start 175.42 59.1754) (end 175.42 76.8339) (width 0.2) (layer "B.Cu") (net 3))
 (segment (start 178.8092 55.7862) (end 175.42 59.1754) (width 0.2) (layer "B.Cu") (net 3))
 (segment (start 177.325 83.6905) (end 170.9005 90.115) (width 0.2) (layer "F.Cu") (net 14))
 (segment (start 180.5 76.6357) (end 177.325 79.8107) (width 0.2) (layer "F.Cu") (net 14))
 (segment (start 170.9005 90.115) (end 169.32 90.115) (width 0.2) (layer "F.Cu") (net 14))
 (segment (start 180.5 73.35) (end 180.5 76.6357) (width 0.2) (layer "F.Cu") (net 14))
 (segment (start 177.325 79.8107) (end 177.325 83.6905) (width 0.2) (layer "F.Cu") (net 14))
 (segment (start 172.7664 78.6367) (end 169.073 78.6367) (width 0.2) (layer "F.Cu") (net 16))
 (segment (start 177.96 73.35) (end 177.96 73.7964) (width 0.2) (layer "F.Cu") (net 16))
 (segment (start 176.505 75.2514) (end 176.1517 75.2514) (width 0.2) (layer "F.Cu") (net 16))
 (segment (start 177.96 73.7964) (end 176.505 75.2514) (width 0.2) (layer "F.Cu") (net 16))
 (segment (start 176.1517 75.2514) (end 172.7664 78.6367) (width 0.2) (layer "F.Cu") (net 16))
 (segment (start 162.8017 85.5094) (end 161.8378 86.4733) (width 0.2) (layer "F.Cu") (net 16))
 (segment (start 161.7 87.575) (end 161.7 86.4733) (width 0.2) (layer "F.Cu") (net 16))
 (segment (start 161.8378 86.4733) (end 161.7 86.4733) (width 0.2) (layer "F.Cu") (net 16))
 (segment (start 162.8017 84.908) (end 162.8017 85.5094) (width 0.2) (layer "F.Cu") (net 16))
 (segment (start 169.073 78.6367) (end 162.8017 84.908) (width 0.2) (layer "F.Cu") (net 16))
 (segment (start 166.3193 79.4731) (end 166.3193 78.7918) (width 0.2) (layer "F.Cu") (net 15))
 (segment (start 180.4935 59.7373) (end 180.8447 60.0885) (width 0.2) (layer "F.Cu") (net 15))
 (segment (start 180.8447 61.9179) (end 179.23 63.5326) (width 0.2) (layer "F.Cu") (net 15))
 (segment (start 168.9661 76.145) (end 174.3418 76.145) (width 0.2) (layer "F.Cu") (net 15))
 (segment (start 161.7 90.115) (end 161.7 89.0133) (width 0.2) (layer "F.Cu") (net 15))
 (segment (start 179.23 63.5326) (end 179.23 73.35) (width 0.2) (layer "F.Cu") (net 15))
 (segment (start 160.5755 84.5206) (end 161.3311 83.765) (width 0.2) (layer "F.Cu") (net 15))
 (segment (start 161.5069 89.0133) (end 160.5755 88.0819) (width 0.2) (layer "F.Cu") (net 15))
 (segment (start 178.5705 59.7373) (end 180.4935 59.7373) (width 0.2) (layer "F.Cu") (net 15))
 (segment (start 176.055 74.4318) (end 176.055 62.2528) (width 0.2) (layer "F.Cu") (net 15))
 (segment (start 176.055 62.2528) (end 178.5705 59.7373) (width 0.2) (layer "F.Cu") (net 15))
 (segment (start 161.7 89.0133) (end 161.5069 89.0133) (width 0.2) (layer "F.Cu") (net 15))
 (segment (start 162.0274 83.765) (end 166.3193 79.4731) (width 0.2) (layer "F.Cu") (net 15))
 (segment (start 174.3418 76.145) (end 176.055 74.4318) (width 0.2) (layer "F.Cu") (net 15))
 (segment (start 166.3193 78.7918) (end 168.9661 76.145) (width 0.2) (layer "F.Cu") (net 15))
 (segment (start 180.8447 60.0885) (end 180.8447 61.9179) (width 0.2) (layer "F.Cu") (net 15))
 (segment (start 161.3311 83.765) (end 162.0274 83.765) (width 0.2) (layer "F.Cu") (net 15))
 (segment (start 160.5755 88.0819) (end 160.5755 84.5206) (width 0.2) (layer "F.Cu") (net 15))
 (segment (start 168.1924 90.5797) (end 168.1924 89.6097) (width 0.2) (layer "F.Cu") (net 13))
 (segment (start 169.32 87.575) (end 169.32 88.6767) (width 0.2) (layer "F.Cu") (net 13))
 (segment (start 171.0946 91.2217) (end 168.8344 91.2217) (width 0.2) (layer "F.Cu") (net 13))
 (segment (start 169.1254 88.6767) (end 169.32 88.6767) (width 0.2) (layer "F.Cu") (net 13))
 (segment (start 168.1924 89.6097) (end 169.1254 88.6767) (width 0.2) (layer "F.Cu") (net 13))
 (segment (start 181.77 73.35) (end 181.77 77.884) (width 0.2) (layer "F.Cu") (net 13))
 (segment (start 181.77 77.884) (end 178.595 81.059) (width 0.2) (layer "F.Cu") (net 13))
 (segment (start 168.8344 91.2217) (end 168.1924 90.5797) (width 0.2) (layer "F.Cu") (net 13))
 (segment (start 178.595 83.7213) (end 171.0946 91.2217) (width 0.2) (layer "F.Cu") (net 13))
 (segment (start 178.595 81.059) (end 178.595 83.7213) (width 0.2) (layer "F.Cu") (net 13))
 (segment (start 178.6017 74.8622) (end 178.6017 61.3283) (width 0.2) (layer "F.Cu") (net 4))
 (segment (start 176.69 76.7739) (end 178.6017 74.8622) (width 0.2) (layer "F.Cu") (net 4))
 (segment (start 178.6017 61.3283) (end 179.525 60.405) (width 0.2) (layer "F.Cu") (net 4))
 (segment (start 176.69 82.65) (end 176.69 76.7739) (width 0.2) (layer "F.Cu") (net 4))
 (segment (start 183.04 73.35) (end 183.04 74.8785) (width 0.2) (layer "F.Cu") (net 12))
 (via (at 183.04 74.8785) (size 0.6) (drill 0.3) (layers "F.Cu" "B.Cu") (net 12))
 (segment (start 161.7 85.035) (end 162.8017 85.035) (width 0.2) (layer "B.Cu") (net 12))
 (segment (start 173.9852 83.9333) (end 183.04 74.8785) (width 0.2) (layer "B.Cu") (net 12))
 (segment (start 163.9034 83.9333) (end 173.9852 83.9333) (width 0.2) (layer "B.Cu") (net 12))
 (segment (start 162.8017 85.035) (end 163.9034 83.9333) (width 0.2) (layer "B.Cu") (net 12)))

